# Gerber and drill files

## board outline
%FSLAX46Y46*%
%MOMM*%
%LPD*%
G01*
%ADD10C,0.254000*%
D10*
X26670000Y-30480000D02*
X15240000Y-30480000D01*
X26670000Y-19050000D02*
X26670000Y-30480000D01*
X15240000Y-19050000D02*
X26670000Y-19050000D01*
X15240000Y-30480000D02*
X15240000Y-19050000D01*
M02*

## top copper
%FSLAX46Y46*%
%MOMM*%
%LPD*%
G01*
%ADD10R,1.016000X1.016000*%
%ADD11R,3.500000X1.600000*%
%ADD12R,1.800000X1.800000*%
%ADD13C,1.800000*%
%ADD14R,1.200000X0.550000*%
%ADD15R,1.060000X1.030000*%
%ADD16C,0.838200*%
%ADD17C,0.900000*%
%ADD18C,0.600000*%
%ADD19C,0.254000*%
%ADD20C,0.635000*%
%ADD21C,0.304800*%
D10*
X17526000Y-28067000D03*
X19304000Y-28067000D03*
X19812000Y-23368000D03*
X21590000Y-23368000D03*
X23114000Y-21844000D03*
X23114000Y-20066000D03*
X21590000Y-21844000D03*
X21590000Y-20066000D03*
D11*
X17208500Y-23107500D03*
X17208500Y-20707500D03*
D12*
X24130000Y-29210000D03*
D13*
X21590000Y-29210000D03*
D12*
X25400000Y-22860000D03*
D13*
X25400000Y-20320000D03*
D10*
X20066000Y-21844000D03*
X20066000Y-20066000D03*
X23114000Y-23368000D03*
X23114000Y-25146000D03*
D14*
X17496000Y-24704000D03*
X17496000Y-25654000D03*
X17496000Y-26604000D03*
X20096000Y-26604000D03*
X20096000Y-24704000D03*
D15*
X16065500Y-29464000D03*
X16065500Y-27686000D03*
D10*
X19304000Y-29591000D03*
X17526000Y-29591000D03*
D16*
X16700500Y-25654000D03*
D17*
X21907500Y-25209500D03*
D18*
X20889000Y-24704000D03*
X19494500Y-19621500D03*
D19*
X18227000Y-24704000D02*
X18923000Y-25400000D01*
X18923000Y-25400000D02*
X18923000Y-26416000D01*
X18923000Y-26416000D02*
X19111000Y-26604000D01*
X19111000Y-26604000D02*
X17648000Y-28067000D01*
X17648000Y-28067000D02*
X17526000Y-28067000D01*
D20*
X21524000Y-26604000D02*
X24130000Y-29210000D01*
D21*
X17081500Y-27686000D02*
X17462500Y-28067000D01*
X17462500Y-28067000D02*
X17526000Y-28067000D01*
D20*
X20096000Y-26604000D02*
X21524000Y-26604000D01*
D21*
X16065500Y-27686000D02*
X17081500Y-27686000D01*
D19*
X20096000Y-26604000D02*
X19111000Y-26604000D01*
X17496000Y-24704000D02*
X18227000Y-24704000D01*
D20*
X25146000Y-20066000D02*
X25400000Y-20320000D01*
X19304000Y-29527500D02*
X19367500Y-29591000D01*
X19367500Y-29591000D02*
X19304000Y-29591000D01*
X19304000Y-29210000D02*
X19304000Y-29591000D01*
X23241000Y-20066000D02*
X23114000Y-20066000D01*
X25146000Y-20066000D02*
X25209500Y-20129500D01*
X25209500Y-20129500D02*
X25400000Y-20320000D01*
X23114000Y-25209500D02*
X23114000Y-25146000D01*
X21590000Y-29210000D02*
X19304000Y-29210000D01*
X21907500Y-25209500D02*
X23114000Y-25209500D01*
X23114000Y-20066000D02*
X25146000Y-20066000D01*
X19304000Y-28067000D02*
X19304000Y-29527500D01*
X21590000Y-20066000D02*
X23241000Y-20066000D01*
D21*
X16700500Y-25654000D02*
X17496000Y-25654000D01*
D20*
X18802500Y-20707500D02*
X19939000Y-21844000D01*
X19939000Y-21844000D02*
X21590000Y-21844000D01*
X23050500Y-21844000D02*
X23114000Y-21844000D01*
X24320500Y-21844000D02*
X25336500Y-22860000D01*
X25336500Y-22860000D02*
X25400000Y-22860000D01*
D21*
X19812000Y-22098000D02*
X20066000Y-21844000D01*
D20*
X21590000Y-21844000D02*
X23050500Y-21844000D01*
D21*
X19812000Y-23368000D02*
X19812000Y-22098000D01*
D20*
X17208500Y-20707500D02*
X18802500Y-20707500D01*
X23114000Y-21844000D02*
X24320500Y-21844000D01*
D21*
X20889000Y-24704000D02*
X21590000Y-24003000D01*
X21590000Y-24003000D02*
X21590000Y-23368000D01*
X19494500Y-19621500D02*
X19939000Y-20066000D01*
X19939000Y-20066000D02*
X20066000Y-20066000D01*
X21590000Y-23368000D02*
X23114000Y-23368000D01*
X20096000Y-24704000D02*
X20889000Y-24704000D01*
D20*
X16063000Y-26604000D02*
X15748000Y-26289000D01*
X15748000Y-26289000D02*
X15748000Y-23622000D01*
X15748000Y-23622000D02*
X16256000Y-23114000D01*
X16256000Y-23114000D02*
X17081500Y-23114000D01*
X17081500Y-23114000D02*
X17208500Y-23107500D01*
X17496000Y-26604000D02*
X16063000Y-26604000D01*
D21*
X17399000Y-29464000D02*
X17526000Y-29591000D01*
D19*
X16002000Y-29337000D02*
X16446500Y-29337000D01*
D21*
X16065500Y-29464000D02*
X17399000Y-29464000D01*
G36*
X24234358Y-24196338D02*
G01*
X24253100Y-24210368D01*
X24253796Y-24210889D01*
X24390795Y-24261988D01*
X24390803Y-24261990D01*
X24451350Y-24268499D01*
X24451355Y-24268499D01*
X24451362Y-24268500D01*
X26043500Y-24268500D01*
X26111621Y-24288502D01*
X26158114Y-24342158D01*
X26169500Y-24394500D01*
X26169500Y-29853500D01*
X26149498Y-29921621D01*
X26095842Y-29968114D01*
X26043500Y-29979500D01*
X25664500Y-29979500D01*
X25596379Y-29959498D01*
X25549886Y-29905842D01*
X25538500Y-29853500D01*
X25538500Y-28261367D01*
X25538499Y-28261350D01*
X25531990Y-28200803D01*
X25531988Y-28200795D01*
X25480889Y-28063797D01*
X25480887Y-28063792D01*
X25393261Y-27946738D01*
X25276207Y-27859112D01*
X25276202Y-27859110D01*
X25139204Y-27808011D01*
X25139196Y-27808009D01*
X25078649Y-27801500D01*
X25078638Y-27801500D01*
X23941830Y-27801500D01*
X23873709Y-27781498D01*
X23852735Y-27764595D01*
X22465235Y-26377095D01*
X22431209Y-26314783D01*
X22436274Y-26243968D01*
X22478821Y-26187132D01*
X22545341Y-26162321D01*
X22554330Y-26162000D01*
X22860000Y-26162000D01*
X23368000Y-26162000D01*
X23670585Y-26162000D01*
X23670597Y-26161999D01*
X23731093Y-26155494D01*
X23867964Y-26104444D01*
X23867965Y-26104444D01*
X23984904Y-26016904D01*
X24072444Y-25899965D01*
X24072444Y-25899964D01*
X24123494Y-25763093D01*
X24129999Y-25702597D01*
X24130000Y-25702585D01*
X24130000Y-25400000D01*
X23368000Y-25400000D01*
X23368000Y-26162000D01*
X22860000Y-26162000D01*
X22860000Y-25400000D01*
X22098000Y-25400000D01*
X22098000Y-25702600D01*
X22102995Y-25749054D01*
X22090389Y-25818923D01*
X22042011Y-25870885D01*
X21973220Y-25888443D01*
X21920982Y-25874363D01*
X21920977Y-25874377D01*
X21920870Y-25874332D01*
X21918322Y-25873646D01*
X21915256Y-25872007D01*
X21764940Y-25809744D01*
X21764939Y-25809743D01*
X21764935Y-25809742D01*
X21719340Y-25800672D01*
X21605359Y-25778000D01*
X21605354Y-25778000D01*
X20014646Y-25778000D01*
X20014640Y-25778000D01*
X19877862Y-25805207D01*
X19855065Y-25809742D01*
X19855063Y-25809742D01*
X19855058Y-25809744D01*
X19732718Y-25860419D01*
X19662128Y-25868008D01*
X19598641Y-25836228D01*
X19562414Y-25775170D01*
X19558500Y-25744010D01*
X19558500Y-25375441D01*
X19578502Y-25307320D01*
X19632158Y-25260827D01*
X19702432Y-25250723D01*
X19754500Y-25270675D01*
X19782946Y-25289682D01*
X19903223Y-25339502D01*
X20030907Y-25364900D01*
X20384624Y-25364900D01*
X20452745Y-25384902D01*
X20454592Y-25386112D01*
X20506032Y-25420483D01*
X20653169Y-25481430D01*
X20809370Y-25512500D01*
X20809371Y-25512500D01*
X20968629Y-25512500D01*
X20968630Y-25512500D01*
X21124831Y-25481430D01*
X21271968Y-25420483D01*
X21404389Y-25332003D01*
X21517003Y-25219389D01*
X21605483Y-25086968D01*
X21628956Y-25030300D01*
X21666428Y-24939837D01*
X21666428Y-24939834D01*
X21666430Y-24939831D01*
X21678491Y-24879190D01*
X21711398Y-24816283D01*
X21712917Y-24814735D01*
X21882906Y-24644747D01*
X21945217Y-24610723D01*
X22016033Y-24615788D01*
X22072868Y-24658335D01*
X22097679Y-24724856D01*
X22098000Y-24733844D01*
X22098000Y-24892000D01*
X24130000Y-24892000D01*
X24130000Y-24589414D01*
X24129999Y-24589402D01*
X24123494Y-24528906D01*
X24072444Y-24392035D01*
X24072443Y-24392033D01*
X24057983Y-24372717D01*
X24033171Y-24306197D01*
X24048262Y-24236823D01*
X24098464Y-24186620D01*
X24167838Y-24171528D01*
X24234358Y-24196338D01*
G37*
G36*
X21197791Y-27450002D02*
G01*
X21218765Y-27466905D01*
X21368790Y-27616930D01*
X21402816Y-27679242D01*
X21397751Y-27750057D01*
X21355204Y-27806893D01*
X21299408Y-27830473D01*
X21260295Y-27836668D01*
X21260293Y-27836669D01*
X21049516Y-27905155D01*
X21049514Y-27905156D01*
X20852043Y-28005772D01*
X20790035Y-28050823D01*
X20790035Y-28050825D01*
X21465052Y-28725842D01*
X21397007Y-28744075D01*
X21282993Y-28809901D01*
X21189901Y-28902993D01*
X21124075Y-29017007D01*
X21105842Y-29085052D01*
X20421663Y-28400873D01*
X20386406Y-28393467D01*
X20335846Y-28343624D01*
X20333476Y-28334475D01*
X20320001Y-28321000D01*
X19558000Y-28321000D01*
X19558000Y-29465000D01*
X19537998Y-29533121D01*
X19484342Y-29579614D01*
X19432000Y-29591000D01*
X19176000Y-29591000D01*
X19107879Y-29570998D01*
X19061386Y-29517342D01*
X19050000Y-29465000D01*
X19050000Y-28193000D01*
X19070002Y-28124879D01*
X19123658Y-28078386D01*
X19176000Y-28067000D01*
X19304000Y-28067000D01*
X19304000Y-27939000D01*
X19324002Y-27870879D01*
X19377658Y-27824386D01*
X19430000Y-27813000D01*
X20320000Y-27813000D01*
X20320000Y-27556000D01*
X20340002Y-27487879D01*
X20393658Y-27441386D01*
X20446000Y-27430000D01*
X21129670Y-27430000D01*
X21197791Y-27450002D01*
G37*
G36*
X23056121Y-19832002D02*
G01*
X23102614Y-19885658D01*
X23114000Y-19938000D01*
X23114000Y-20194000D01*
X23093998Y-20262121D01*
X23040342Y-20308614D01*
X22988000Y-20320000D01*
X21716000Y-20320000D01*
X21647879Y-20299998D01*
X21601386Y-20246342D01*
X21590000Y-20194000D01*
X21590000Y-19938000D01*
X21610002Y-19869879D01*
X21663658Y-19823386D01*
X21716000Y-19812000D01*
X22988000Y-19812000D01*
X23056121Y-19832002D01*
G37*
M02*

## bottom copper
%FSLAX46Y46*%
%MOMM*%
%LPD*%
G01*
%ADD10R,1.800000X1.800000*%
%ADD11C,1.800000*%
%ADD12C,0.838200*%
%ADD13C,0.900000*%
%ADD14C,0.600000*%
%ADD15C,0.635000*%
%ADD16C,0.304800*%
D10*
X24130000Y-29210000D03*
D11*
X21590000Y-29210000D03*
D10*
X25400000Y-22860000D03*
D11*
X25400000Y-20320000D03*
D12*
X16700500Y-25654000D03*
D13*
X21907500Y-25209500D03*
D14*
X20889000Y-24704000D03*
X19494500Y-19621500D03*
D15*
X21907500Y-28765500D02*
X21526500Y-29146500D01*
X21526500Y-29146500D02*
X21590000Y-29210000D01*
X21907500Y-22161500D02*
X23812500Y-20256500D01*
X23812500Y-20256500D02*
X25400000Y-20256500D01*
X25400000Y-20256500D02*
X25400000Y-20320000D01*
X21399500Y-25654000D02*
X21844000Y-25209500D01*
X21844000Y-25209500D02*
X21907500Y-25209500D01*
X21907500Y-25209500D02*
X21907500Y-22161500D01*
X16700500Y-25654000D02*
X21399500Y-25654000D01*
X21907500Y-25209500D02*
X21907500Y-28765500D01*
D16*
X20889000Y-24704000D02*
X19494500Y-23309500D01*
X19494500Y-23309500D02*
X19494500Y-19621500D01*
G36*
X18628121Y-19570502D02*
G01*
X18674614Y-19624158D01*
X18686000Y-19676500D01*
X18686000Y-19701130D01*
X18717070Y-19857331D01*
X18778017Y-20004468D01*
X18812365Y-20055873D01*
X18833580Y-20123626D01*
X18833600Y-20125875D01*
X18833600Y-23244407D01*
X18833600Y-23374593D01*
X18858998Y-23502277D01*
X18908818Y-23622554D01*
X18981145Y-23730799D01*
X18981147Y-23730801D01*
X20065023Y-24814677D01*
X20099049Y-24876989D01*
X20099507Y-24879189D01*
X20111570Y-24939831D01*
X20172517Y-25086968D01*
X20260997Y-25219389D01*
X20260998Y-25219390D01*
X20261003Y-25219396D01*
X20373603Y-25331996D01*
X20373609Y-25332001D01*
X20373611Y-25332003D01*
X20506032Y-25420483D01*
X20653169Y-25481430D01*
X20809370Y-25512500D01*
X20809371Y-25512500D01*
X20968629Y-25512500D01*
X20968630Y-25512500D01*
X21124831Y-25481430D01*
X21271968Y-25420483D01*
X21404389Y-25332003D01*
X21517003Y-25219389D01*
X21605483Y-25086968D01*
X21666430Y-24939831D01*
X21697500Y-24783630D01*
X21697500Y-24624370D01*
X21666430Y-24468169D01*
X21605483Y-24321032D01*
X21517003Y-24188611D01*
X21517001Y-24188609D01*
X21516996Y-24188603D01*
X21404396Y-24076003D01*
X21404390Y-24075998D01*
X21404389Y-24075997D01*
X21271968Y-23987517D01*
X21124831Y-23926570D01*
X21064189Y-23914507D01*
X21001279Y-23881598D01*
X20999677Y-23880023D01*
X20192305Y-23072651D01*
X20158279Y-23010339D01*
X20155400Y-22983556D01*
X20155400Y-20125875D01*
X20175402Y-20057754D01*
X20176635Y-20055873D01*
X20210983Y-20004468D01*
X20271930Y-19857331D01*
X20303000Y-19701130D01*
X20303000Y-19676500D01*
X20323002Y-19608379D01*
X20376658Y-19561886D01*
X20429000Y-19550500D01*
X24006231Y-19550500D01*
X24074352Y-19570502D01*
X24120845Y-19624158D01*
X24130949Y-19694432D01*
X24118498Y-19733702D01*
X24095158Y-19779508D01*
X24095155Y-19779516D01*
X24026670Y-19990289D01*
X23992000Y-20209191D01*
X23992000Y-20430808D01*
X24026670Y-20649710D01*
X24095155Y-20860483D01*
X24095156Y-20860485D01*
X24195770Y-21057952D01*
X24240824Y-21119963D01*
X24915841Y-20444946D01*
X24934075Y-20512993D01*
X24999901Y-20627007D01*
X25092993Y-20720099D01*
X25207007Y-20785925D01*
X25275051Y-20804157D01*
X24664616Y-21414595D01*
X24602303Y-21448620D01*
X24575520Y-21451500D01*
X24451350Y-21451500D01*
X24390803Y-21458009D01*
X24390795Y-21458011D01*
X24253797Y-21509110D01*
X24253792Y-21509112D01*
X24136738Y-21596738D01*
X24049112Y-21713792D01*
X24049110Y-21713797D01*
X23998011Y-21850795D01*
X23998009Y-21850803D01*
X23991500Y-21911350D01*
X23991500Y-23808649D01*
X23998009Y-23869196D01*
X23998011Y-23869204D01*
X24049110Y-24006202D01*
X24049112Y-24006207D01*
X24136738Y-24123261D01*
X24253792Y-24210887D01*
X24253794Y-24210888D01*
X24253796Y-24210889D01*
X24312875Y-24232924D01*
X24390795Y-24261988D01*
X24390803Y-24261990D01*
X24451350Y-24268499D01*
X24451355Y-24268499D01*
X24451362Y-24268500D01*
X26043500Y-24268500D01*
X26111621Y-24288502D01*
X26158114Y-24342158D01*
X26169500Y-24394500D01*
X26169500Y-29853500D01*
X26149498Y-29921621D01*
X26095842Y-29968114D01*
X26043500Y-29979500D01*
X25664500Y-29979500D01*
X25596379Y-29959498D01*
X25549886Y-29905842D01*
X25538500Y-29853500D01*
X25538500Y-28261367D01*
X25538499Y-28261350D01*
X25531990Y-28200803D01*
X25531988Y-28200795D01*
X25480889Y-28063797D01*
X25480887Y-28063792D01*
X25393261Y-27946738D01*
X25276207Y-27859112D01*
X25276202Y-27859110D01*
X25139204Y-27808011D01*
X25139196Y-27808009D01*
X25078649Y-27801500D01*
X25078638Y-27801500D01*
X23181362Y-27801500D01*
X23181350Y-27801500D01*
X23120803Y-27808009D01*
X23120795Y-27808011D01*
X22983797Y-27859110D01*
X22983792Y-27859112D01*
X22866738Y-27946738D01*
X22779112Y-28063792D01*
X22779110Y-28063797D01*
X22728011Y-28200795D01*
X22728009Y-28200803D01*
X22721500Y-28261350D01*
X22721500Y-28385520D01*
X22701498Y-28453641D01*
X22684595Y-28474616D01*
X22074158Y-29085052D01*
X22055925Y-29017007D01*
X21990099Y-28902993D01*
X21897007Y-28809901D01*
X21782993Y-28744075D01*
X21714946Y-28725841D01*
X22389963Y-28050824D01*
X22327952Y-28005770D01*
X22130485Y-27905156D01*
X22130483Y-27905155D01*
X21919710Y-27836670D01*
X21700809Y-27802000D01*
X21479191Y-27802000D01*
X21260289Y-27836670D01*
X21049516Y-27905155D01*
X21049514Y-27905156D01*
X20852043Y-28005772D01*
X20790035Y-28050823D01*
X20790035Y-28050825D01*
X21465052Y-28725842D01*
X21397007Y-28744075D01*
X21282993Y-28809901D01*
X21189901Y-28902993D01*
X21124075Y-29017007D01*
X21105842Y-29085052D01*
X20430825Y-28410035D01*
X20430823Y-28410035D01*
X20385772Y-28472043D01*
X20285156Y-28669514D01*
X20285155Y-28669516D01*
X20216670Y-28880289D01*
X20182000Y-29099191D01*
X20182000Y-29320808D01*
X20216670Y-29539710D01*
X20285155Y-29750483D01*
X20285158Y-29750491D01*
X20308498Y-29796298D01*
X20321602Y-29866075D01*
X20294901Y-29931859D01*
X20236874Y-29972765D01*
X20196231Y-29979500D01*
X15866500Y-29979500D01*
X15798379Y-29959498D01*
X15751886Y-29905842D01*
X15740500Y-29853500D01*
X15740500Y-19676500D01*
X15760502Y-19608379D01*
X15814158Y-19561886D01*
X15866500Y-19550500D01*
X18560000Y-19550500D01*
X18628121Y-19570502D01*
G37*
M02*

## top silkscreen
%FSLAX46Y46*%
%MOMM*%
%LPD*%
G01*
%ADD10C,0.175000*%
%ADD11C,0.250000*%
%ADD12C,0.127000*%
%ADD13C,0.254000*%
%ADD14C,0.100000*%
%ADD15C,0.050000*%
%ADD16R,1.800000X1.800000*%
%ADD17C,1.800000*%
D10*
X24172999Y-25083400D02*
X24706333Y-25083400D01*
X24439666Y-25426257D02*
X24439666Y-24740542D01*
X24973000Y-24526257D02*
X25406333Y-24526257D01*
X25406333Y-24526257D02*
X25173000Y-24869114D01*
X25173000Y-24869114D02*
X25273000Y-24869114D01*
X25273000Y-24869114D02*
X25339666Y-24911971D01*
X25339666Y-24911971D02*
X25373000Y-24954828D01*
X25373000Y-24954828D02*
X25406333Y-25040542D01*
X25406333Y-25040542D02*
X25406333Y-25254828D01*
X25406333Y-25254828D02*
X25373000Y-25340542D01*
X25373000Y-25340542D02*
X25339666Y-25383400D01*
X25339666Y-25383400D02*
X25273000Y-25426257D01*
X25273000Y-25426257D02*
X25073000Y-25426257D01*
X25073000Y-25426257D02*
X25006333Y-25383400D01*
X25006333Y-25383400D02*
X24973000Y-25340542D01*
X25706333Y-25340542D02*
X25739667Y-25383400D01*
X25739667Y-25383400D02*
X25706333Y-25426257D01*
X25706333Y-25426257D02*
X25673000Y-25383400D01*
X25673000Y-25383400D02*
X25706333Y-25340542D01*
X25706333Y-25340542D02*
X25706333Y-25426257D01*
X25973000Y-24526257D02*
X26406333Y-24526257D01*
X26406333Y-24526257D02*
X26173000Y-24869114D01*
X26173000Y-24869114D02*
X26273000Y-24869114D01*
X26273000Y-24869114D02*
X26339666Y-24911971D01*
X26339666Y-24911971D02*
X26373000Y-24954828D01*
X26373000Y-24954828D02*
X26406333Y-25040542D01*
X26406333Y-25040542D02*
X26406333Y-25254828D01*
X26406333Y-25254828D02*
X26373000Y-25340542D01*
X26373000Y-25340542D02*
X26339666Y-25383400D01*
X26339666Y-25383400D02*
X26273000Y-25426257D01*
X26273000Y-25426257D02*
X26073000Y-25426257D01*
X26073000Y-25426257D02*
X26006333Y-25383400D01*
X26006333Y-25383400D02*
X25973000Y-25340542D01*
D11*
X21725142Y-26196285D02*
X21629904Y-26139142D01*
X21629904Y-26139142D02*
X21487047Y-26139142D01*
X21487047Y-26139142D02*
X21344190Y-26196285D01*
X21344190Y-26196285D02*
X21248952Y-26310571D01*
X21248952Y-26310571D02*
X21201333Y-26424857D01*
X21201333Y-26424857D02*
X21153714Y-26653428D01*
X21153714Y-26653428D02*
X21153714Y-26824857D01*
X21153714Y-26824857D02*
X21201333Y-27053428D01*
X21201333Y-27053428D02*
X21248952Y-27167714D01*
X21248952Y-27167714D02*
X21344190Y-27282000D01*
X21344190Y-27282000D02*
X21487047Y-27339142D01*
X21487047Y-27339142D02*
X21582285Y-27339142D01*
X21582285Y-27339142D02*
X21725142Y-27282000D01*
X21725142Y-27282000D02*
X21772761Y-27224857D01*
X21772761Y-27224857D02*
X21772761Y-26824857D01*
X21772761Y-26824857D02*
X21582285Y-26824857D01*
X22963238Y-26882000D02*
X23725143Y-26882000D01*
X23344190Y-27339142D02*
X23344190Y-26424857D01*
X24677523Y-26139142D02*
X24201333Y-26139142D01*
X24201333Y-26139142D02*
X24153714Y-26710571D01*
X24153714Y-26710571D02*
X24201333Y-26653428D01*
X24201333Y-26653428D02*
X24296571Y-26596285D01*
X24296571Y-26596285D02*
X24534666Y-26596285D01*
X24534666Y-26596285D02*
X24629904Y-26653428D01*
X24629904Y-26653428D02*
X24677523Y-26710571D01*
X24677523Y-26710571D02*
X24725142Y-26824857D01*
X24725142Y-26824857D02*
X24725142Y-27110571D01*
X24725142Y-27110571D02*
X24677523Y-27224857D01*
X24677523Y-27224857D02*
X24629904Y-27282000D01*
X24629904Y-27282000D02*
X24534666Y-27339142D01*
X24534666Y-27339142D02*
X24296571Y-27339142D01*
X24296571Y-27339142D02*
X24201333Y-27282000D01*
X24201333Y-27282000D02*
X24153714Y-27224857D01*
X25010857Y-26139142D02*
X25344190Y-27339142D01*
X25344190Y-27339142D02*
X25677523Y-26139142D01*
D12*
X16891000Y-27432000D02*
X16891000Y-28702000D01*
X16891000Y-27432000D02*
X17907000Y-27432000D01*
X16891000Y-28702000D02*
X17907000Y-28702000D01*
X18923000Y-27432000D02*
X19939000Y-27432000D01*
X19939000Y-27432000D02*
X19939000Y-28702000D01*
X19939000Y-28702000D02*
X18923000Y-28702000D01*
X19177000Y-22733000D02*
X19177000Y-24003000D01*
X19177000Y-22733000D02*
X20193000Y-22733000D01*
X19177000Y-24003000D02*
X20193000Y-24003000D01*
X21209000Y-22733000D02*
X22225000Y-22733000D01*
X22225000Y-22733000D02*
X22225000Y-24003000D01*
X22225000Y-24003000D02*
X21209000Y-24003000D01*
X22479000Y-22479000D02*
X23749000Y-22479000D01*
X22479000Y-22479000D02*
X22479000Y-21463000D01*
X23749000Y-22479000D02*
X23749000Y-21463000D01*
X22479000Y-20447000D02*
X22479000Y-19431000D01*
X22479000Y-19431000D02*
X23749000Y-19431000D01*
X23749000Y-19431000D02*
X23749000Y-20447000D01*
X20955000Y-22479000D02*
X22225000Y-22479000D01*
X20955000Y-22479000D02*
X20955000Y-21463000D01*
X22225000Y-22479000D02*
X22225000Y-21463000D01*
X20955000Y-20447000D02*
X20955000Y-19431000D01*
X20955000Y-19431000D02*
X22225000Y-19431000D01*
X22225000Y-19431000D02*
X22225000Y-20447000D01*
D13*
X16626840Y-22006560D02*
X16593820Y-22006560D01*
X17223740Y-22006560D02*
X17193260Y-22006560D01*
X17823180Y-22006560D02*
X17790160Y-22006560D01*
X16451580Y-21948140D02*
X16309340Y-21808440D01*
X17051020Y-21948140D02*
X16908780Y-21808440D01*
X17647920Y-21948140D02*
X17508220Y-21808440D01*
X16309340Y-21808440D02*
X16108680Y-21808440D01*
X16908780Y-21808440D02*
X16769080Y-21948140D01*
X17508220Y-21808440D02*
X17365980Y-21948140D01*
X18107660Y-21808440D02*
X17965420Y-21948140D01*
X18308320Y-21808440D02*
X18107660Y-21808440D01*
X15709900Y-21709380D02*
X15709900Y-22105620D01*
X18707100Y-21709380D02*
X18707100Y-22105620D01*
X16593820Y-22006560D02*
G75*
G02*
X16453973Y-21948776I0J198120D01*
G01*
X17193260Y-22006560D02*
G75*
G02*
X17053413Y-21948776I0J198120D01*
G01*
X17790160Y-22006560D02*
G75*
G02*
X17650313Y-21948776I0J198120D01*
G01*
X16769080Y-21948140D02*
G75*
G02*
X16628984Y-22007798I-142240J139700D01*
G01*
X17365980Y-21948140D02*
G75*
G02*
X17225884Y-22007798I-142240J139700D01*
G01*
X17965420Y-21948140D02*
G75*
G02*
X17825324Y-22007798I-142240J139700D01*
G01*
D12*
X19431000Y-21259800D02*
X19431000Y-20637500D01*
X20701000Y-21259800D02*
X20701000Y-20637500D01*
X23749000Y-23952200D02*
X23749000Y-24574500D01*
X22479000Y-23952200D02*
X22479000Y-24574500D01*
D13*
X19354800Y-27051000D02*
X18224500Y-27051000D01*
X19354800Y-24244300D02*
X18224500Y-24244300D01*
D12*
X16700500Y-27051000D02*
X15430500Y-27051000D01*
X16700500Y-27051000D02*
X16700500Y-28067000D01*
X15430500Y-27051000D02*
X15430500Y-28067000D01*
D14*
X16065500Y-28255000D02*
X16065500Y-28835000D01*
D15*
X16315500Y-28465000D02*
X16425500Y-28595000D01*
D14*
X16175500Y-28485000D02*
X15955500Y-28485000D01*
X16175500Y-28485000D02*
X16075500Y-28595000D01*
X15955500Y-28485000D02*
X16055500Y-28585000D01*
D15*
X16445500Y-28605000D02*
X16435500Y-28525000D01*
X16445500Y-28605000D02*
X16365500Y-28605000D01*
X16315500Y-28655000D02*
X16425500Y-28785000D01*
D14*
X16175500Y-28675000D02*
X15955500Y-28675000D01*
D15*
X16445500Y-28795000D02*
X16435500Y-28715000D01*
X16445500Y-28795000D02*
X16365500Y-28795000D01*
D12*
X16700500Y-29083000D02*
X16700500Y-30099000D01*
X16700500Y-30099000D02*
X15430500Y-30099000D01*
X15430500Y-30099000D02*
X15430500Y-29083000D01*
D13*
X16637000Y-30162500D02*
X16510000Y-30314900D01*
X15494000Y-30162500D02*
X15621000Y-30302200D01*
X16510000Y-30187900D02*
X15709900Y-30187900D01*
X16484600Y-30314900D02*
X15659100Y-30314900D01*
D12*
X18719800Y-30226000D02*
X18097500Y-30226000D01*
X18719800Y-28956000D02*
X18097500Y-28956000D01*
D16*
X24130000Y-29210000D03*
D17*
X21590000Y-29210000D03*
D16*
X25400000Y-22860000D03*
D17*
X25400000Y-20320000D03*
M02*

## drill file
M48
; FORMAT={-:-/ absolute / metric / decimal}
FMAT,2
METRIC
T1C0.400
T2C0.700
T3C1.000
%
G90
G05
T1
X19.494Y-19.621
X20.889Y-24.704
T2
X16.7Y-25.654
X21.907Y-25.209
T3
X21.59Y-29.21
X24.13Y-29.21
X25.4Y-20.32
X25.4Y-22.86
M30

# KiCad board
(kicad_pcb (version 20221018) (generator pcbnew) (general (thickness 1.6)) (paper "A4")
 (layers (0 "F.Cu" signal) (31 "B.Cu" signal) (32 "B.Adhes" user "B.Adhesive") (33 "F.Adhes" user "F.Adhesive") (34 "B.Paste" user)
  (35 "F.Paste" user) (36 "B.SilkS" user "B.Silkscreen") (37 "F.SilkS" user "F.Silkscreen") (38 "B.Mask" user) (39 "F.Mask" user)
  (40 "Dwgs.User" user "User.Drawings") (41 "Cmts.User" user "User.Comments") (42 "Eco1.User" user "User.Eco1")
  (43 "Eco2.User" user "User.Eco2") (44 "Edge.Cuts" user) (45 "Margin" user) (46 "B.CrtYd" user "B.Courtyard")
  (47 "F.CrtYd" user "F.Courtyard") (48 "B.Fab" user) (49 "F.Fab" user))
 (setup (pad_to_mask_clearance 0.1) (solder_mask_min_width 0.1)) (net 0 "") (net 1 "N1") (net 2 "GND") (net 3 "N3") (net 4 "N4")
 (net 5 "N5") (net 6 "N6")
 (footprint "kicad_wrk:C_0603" (layer "F.Cu") (at 18.415 28.067)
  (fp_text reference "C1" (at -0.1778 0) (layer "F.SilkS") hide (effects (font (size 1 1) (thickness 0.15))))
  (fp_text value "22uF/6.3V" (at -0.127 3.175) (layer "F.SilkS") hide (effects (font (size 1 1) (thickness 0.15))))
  (fp_line (start -1.524 -0.635) (end -1.524 0.635) (stroke (width 0.127) (type solid)) (layer "F.SilkS"))
  (fp_line (start -1.524 -0.635) (end -0.508 -0.635) (stroke (width 0.127) (type solid)) (layer "F.SilkS"))
  (fp_line (start -1.524 0.635) (end -0.508 0.635) (stroke (width 0.127) (type solid)) (layer "F.SilkS"))
  (fp_line (start 0.508 -0.635) (end 1.524 -0.635) (stroke (width 0.127) (type solid)) (layer "F.SilkS"))
  (fp_line (start 1.524 -0.635) (end 1.524 0.635) (stroke (width 0.127) (type solid)) (layer "F.SilkS"))
  (fp_line (start 1.524 0.635) (end 0.508 0.635) (stroke (width 0.127) (type solid)) (layer "F.SilkS"))
  (pad "1" smd rect (at -0.889 0) (size 1.016 1.016) (layers "F.Cu" "F.Paste" "F.Mask") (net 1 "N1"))
  (pad "2" smd rect (at 0.889 0) (size 1.016 1.016) (layers "F.Cu" "F.Paste" "F.Mask") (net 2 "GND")))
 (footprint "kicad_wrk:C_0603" (layer "F.Cu") (at 20.701 23.368)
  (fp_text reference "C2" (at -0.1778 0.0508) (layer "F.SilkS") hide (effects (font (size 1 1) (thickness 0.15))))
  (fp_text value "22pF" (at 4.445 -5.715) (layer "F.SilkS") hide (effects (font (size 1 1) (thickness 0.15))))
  (fp_line (start -1.524 -0.635) (end -1.524 0.635) (stroke (width 0.127) (type solid)) (layer "F.SilkS"))
  (fp_line (start -1.524 -0.635) (end -0.508 -0.635) (stroke (width 0.127) (type solid)) (layer "F.SilkS"))
  (fp_line (start -1.524 0.635) (end -0.508 0.635) (stroke (width 0.127) (type solid)) (layer "F.SilkS"))
  (fp_line (start 0.508 -0.635) (end 1.524 -0.635) (stroke (width 0.127) (type solid)) (layer "F.SilkS"))
  (fp_line (start 1.524 -0.635) (end 1.524 0.635) (stroke (width 0.127) (type solid)) (layer "F.SilkS"))
  (fp_line (start 1.524 0.635) (end 0.508 0.635) (stroke (width 0.127) (type solid)) (layer "F.SilkS"))
  (pad "1" smd rect (at -0.889 0) (size 1.016 1.016) (layers "F.Cu" "F.Paste" "F.Mask") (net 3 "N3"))
  (pad "2" smd rect (at 0.889 0) (size 1.016 1.016) (layers "F.Cu" "F.Paste" "F.Mask") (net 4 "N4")))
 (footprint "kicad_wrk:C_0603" (layer "F.Cu") (at 23.114 20.955 90)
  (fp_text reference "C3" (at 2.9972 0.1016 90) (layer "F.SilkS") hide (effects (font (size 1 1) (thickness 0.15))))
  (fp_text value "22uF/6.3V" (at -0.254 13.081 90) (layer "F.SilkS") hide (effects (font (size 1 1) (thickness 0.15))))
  (fp_line (start -1.524 -0.635) (end -1.524 0.635) (stroke (width 0.127) (type solid)) (layer "F.SilkS"))
  (fp_line (start -1.524 -0.635) (end -0.508 -0.635) (stroke (width 0.127) (type solid)) (layer "F.SilkS"))
  (fp_line (start -1.524 0.635) (end -0.508 0.635) (stroke (width 0.127) (type solid)) (layer "F.SilkS"))
  (fp_line (start 0.508 -0.635) (end 1.524 -0.635) (stroke (width 0.127) (type solid)) (layer "F.SilkS"))
  (fp_line (start 1.524 -0.635) (end 1.524 0.635) (stroke (width 0.127) (type solid)) (layer "F.SilkS"))
  (fp_line (start 1.524 0.635) (end 0.508 0.635) (stroke (width 0.127) (type solid)) (layer "F.SilkS"))
  (pad "1" smd rect (at -0.889 0 90) (size 1.016 1.016) (layers "F.Cu" "F.Paste" "F.Mask") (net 3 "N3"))
  (pad "2" smd rect (at 0.889 0 90) (size 1.016 1.016) (layers "F.Cu" "F.Paste" "F.Mask") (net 2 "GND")))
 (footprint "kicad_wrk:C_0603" (layer "F.Cu") (at 21.59 20.955 90)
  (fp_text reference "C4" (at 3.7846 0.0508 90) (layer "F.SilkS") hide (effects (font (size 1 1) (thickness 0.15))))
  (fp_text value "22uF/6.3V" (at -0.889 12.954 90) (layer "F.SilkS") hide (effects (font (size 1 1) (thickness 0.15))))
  (fp_line (start -1.524 -0.635) (end -1.524 0.635) (stroke (width 0.127) (type solid)) (layer "F.SilkS"))
  (fp_line (start -1.524 -0.635) (end -0.508 -0.635) (stroke (width 0.127) (type solid)) (layer "F.SilkS"))
  (fp_line (start -1.524 0.635) (end -0.508 0.635) (stroke (width 0.127) (type solid)) (layer "F.SilkS"))
  (fp_line (start 0.508 -0.635) (end 1.524 -0.635) (stroke (width 0.127) (type solid)) (layer "F.SilkS"))
  (fp_line (start 1.524 -0.635) (end 1.524 0.635) (stroke (width 0.127) (type solid)) (layer "F.SilkS"))
  (fp_line (start 1.524 0.635) (end 0.508 0.635) (stroke (width 0.127) (type solid)) (layer "F.SilkS"))
  (pad "1" smd rect (at -0.889 0 90) (size 1.016 1.016) (layers "F.Cu" "F.Paste" "F.Mask") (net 3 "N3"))
  (pad "2" smd rect (at 0.889 0 90) (size 1.016 1.016) (layers "F.Cu" "F.Paste" "F.Mask") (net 2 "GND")))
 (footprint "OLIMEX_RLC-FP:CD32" (layer "F.Cu") (at 17.2085 21.9075 90)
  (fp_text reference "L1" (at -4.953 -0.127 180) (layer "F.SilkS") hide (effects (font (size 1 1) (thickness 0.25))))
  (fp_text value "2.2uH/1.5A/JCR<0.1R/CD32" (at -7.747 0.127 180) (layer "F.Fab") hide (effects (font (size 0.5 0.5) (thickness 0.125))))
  (fp_line (start -0.09906 -0.58166) (end -0.09906 -0.61468) (stroke (width 0.254) (type solid)) (layer "F.SilkS"))
  (fp_line (start -0.09906 0.01524) (end -0.09906 -0.01524) (stroke (width 0.254) (type solid)) (layer "F.SilkS"))
  (fp_line (start -0.09906 0.61468) (end -0.09906 0.58166) (stroke (width 0.254) (type solid)) (layer "F.SilkS"))
  (fp_line (start -0.04064 -0.75692) (end 0.09906 -0.89916) (stroke (width 0.254) (type solid)) (layer "F.SilkS"))
  (fp_line (start -0.04064 -0.15748) (end 0.09906 -0.29972) (stroke (width 0.254) (type solid)) (layer "F.SilkS"))
  (fp_line (start -0.04064 0.43942) (end 0.09906 0.29972) (stroke (width 0.254) (type solid)) (layer "F.SilkS"))
  (fp_line (start 0.09906 -0.89916) (end 0.09906 -1.09982) (stroke (width 0.254) (type solid)) (layer "F.SilkS"))
  (fp_line (start 0.09906 -0.29972) (end -0.04064 -0.43942) (stroke (width 0.254) (type solid)) (layer "F.SilkS"))
  (fp_line (start 0.09906 0.29972) (end -0.04064 0.15748) (stroke (width 0.254) (type solid)) (layer "F.SilkS"))
  (fp_line (start 0.09906 0.89916) (end -0.04064 0.75692) (stroke (width 0.254) (type solid)) (layer "F.SilkS"))
  (fp_line (start 0.09906 1.09982) (end 0.09906 0.89916) (stroke (width 0.254) (type solid)) (layer "F.SilkS"))
  (fp_line (start 0.19812 -1.4986) (end -0.19812 -1.4986) (stroke (width 0.254) (type solid)) (layer "F.SilkS"))
  (fp_line (start 0.19812 1.4986) (end -0.19812 1.4986) (stroke (width 0.254) (type solid)) (layer "F.SilkS"))
  (fp_arc (start -0.09906 -0.61468) (mid -0.084045 -0.690337) (end -0.041276 -0.754527) (stroke (width 0.254) (type solid))
   (layer "F.SilkS"))
  (fp_arc (start -0.09906 -0.01524) (mid -0.084045 -0.090897) (end -0.041276 -0.155087) (stroke (width 0.254) (type solid))
   (layer "F.SilkS"))
  (fp_arc (start -0.09906 0.58166) (mid -0.084045 0.506003) (end -0.041276 0.441813) (stroke (width 0.254) (type solid)) (layer "F.SilkS"))
  (fp_arc (start -0.04064 -0.43942) (mid -0.084371 -0.503548) (end -0.100298 -0.579516) (stroke (width 0.254) (type solid))
   (layer "F.SilkS"))
  (fp_arc (start -0.04064 0.15748) (mid -0.084371 0.093352) (end -0.100298 0.017384) (stroke (width 0.254) (type solid)) (layer "F.SilkS"))
  (fp_arc (start -0.04064 0.75692) (mid -0.084371 0.692792) (end -0.100298 0.616824) (stroke (width 0.254) (type solid)) (layer "F.SilkS"))
  (pad "1" smd rect (at -1.2 0 180) (size 3.5 1.6) (layers "F.Cu" "F.Paste" "F.Mask") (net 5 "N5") (solder_mask_margin 0.0508)
   (solder_paste_margin -0.0508) (clearance 0.0508))
  (pad "2" smd rect (at 1.2 0 180) (size 3.5 1.6) (layers "F.Cu" "F.Paste" "F.Mask") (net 3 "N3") (solder_mask_margin 0.0508)
   (solder_paste_margin -0.0508) (clearance 0.0508)))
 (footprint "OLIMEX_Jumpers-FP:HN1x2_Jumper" (layer "F.Cu") (at 22.86 29.21 180)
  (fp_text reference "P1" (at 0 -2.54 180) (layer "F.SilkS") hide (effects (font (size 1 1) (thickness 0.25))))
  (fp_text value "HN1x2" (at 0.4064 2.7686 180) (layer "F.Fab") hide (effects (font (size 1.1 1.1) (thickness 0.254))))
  (pad "1" thru_hole rect (at -1.27 0 270) (size 1.8 1.8) (drill 1) (layers "*.Cu" "*.Mask" "F.SilkS") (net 1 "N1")
   (solder_mask_margin 0.0508) (solder_paste_margin -0.0508))
  (pad "2" thru_hole circle (at 1.27 0 270) (size 1.8 1.8) (drill 1) (layers "*.Cu" "*.Mask" "F.SilkS") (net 2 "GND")
   (solder_mask_margin 0.0508) (solder_paste_margin -0.0508)))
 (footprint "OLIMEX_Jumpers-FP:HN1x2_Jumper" (layer "F.Cu") (at 25.4 21.59 90)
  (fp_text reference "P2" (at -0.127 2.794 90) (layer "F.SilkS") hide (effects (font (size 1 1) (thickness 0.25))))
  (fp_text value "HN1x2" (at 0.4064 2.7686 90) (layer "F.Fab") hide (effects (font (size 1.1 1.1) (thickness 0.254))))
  (pad "1" thru_hole rect (at -1.27 0 180) (size 1.8 1.8) (drill 1) (layers "*.Cu" "*.Mask" "F.SilkS") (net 3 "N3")
   (solder_mask_margin 0.0508) (solder_paste_margin -0.0508))
  (pad "2" thru_hole circle (at 1.27 0 180) (size 1.8 1.8) (drill 1) (layers "*.Cu" "*.Mask" "F.SilkS") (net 2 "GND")
   (solder_mask_margin 0.0508) (solder_paste_margin -0.0508)))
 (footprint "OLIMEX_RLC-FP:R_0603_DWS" (layer "F.Cu") (at 20.066 20.955 90)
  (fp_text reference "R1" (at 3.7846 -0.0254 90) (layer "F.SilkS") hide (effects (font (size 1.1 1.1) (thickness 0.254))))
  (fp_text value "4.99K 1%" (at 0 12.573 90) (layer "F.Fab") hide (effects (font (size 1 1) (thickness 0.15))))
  (fp_line (start -0.3048 -0.635) (end 0.3175 -0.635) (stroke (width 0.127) (type solid)) (layer "F.SilkS"))
  (fp_line (start -0.3048 0.635) (end 0.3175 0.635) (stroke (width 0.127) (type solid)) (layer "F.SilkS"))
  (pad "1" smd rect (at -0.889 0 90) (size 1.016 1.016) (layers "F.Cu" "F.Paste" "F.Mask") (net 3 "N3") (solder_mask_margin 0.0508)
   (solder_paste_margin -0.0508) (clearance 0.0508))
  (pad "2" smd rect (at 0.889 0 90) (size 1.016 1.016) (layers "F.Cu" "F.Paste" "F.Mask") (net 4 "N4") (solder_mask_margin 0.0508)
   (solder_paste_margin -0.0508) (clearance 0.0508)))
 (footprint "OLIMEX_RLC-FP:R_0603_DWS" (layer "F.Cu") (at 23.114 24.257 -90)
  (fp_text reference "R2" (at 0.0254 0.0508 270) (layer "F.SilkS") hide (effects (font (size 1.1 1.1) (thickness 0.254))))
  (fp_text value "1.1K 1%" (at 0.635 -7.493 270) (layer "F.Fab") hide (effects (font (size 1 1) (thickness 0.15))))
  (fp_line (start -0.3048 -0.635) (end 0.3175 -0.635) (stroke (width 0.127) (type solid)) (layer "F.SilkS"))
  (fp_line (start -0.3048 0.635) (end 0.3175 0.635) (stroke (width 0.127) (type solid)) (layer "F.SilkS"))
  (pad "1" smd rect (at -0.889 0 270) (size 1.016 1.016) (layers "F.Cu" "F.Paste" "F.Mask") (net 4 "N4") (solder_mask_margin 0.0508)
   (solder_paste_margin -0.0508) (clearance 0.0508))
  (pad "2" smd rect (at 0.889 0 270) (size 1.016 1.016) (layers "F.Cu" "F.Paste" "F.Mask") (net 2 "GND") (solder_mask_margin 0.0508)
   (solder_paste_margin -0.0508) (clearance 0.0508)))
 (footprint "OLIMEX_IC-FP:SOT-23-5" (layer "F.Cu") (at 18.796 25.654 180)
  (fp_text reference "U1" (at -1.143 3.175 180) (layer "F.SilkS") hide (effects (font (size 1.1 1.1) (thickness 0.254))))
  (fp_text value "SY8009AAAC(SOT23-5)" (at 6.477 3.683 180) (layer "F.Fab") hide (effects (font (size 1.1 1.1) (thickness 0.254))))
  (fp_line (start -0.5588 -1.397) (end 0.5715 -1.397) (stroke (width 0.254) (type solid)) (layer "F.SilkS"))
  (fp_line (start -0.5588 1.4097) (end 0.5715 1.4097) (stroke (width 0.254) (type solid)) (layer "F.SilkS"))
  (pad "1" smd rect (at 1.3 0.95 180) (size 1.2 0.55) (layers "F.Cu" "F.Paste" "F.Mask") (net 1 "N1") (solder_mask_margin 0.0508)
   (solder_paste_margin -0.0508) (clearance 0.0508))
  (pad "2" smd rect (at 1.3 0 180) (size 1.2 0.55) (layers "F.Cu" "F.Paste" "F.Mask") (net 2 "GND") (solder_mask_margin 0.0508)
   (solder_paste_margin -0.0508) (clearance 0.0508))
  (pad "3" smd rect (at 1.3 -0.95 180) (size 1.2 0.55) (layers "F.Cu" "F.Paste" "F.Mask") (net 5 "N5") (solder_mask_margin 0.0508)
   (solder_paste_margin -0.0508) (clearance 0.0508))
  (pad "4" smd rect (at -1.3 -0.95 180) (size 1.2 0.55) (layers "F.Cu" "F.Paste" "F.Mask") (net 1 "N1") (solder_mask_margin 0.0508)
   (solder_paste_margin -0.0508) (clearance 0.0508))
  (pad "5" smd rect (at -1.3 0.95 180) (size 1.2 0.55) (layers "F.Cu" "F.Paste" "F.Mask") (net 4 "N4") (solder_mask_margin 0.0508)
   (solder_paste_margin -0.0508) (clearance 0.0508)))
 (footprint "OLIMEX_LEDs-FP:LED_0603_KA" (layer "F.Cu") (at 16.0655 28.575 -90)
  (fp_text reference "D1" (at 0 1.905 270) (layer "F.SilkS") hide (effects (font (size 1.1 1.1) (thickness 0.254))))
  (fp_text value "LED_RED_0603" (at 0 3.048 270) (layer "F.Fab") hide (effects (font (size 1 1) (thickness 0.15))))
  (fp_line (start -1.524 -0.635) (end -1.524 0.635) (stroke (width 0.127) (type solid)) (layer "F.SilkS"))
  (fp_line (start -1.524 -0.635) (end -0.508 -0.635) (stroke (width 0.127) (type solid)) (layer "F.SilkS"))
  (fp_line (start -1.524 0.635) (end -0.508 0.635) (stroke (width 0.127) (type solid)) (layer "F.SilkS"))
  (fp_line (start -0.32 0) (end 0.26 0) (stroke (width 0.1) (type solid)) (layer "F.SilkS"))
  (fp_line (start -0.11 -0.25) (end 0.02 -0.36) (stroke (width 0.05) (type solid)) (layer "F.SilkS"))
  (fp_line (start -0.09 -0.11) (end -0.09 0.11) (stroke (width 0.1) (type solid)) (layer "F.SilkS"))
  (fp_line (start -0.09 -0.11) (end 0.02 -0.01) (stroke (width 0.1) (type solid)) (layer "F.SilkS"))
  (fp_line (start -0.09 0.11) (end 0.01 0.01) (stroke (width 0.1) (type solid)) (layer "F.SilkS"))
  (fp_line (start 0.03 -0.38) (end -0.05 -0.37) (stroke (width 0.05) (type solid)) (layer "F.SilkS"))
  (fp_line (start 0.03 -0.38) (end 0.03 -0.3) (stroke (width 0.05) (type solid)) (layer "F.SilkS"))
  (fp_line (start 0.08 -0.25) (end 0.21 -0.36) (stroke (width 0.05) (type solid)) (layer "F.SilkS"))
  (fp_line (start 0.1 -0.11) (end 0.1 0.11) (stroke (width 0.1) (type solid)) (layer "F.SilkS"))
  (fp_line (start 0.22 -0.38) (end 0.14 -0.37) (stroke (width 0.05) (type solid)) (layer "F.SilkS"))
  (fp_line (start 0.22 -0.38) (end 0.22 -0.3) (stroke (width 0.05) (type solid)) (layer "F.SilkS"))
  (fp_line (start 0.508 -0.635) (end 1.524 -0.635) (stroke (width 0.127) (type solid)) (layer "F.SilkS"))
  (fp_line (start 1.524 -0.635) (end 1.524 0.635) (stroke (width 0.127) (type solid)) (layer "F.SilkS"))
  (fp_line (start 1.524 0.635) (end 0.508 0.635) (stroke (width 0.127) (type solid)) (layer "F.SilkS"))
  (fp_line (start 1.5875 -0.5715) (end 1.7399 -0.4445) (stroke (width 0.254) (type solid)) (layer "F.SilkS"))
  (fp_line (start 1.5875 0.5715) (end 1.7272 0.4445) (stroke (width 0.254) (type solid)) (layer "F.SilkS"))
  (fp_line (start 1.6129 -0.4445) (end 1.6129 0.3556) (stroke (width 0.254) (type solid)) (layer "F.SilkS"))
  (fp_line (start 1.7399 -0.4191) (end 1.7399 0.4064) (stroke (width 0.254) (type solid)) (layer "F.SilkS"))
  (pad "1" smd rect (at 0.889 0 270) (size 1.03 1.06) (layers "F.Cu" "F.Paste" "F.Mask") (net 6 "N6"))
  (pad "2" smd rect (at -0.889 0 270) (size 1.03 1.06) (layers "F.Cu" "F.Paste" "F.Mask") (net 1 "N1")))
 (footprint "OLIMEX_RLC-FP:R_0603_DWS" (layer "F.Cu") (at 18.415 29.591 180)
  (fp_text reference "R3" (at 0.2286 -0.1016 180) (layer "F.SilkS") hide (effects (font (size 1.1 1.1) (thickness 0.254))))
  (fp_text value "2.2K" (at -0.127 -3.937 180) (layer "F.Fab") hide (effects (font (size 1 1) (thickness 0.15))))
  (fp_line (start -0.3048 -0.635) (end 0.3175 -0.635) (stroke (width 0.127) (type solid)) (layer "F.SilkS"))
  (fp_line (start -0.3048 0.635) (end 0.3175 0.635) (stroke (width 0.127) (type solid)) (layer "F.SilkS"))
  (pad "1" smd rect (at -0.889 0 180) (size 1.016 1.016) (layers "F.Cu" "F.Paste" "F.Mask") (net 2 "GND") (solder_mask_margin 0.0508)
   (solder_paste_margin -0.0508) (clearance 0.0508))
  (pad "2" smd rect (at 0.889 0 180) (size 1.016 1.016) (layers "F.Cu" "F.Paste" "F.Mask") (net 6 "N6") (solder_mask_margin 0.0508)
   (solder_paste_margin -0.0508) (clearance 0.0508)))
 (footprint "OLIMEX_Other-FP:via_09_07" (layer "F.Cu") (at 16.7005 25.654)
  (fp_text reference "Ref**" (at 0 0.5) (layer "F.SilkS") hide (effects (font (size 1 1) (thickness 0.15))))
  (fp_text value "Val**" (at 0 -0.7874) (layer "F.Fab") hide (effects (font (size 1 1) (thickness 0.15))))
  (pad "0" thru_hole circle (at 0 0) (size 0.8382 0.8382) (drill 0.7) (layers "*.Cu") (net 2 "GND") (zone_connect 2)))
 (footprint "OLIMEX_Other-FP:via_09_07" (layer "F.Cu") (at 21.9075 25.273)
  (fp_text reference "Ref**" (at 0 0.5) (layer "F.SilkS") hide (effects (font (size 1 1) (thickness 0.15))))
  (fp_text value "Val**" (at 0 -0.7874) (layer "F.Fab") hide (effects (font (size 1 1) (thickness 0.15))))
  (pad "0" thru_hole circle (at 0 -0.0635) (size 0.9 0.9) (drill 0.7) (layers "*.Cu") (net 2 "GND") (zone_connect 2)))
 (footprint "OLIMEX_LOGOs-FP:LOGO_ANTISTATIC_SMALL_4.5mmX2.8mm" (layer "B.Cu") (at 18.4785 28.194 180)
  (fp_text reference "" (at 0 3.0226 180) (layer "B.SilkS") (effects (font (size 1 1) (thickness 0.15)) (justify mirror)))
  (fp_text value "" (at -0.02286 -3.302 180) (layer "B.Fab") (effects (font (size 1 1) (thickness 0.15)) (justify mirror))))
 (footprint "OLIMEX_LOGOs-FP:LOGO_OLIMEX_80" (layer "B.Cu") (at 19.939 24.3205 180)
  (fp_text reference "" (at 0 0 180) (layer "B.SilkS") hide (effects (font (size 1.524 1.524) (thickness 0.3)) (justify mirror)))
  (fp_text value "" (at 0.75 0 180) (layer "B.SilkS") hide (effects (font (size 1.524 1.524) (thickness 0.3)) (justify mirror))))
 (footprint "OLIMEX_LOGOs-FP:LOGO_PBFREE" (layer "B.Cu") (at 18.669 21.3995 180)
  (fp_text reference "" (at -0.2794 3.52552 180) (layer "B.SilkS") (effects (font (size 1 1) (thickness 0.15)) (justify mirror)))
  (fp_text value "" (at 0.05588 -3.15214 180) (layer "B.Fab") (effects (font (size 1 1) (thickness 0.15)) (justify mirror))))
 (gr_line (start 26.67 30.48) (end 15.24 30.48) (stroke (width 0.254) (type solid)) (layer "Edge.Cuts"))
 (gr_line (start 26.67 19.05) (end 26.67 30.48) (stroke (width 0.254) (type solid)) (layer "Edge.Cuts"))
 (gr_line (start 15.24 19.05) (end 26.67 19.05) (stroke (width 0.254) (type solid)) (layer "Edge.Cuts"))
 (gr_line (start 15.24 30.48) (end 15.24 19.05) (stroke (width 0.254) (type solid)) (layer "Edge.Cuts"))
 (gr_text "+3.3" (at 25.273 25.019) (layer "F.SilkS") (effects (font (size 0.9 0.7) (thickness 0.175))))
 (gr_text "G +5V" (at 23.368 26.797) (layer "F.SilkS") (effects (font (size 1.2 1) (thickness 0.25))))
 (segment (start 18.227 24.704) (end 18.923 25.4) (width 0.254) (layer "F.Cu") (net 1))
 (segment (start 18.923 25.4) (end 18.923 26.416) (width 0.254) (layer "F.Cu") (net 1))
 (segment (start 18.923 26.416) (end 19.111 26.604) (width 0.254) (layer "F.Cu") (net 1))
 (segment (start 19.111 26.604) (end 17.648 28.067) (width 0.254) (layer "F.Cu") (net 1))
 (segment (start 17.648 28.067) (end 17.526 28.067) (width 0.254) (layer "F.Cu") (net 1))
 (segment (start 21.524 26.604) (end 24.13 29.21) (width 0.635) (layer "F.Cu") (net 1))
 (segment (start 17.0815 27.686) (end 17.4625 28.067) (width 0.3048) (layer "F.Cu") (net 1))
 (segment (start 17.4625 28.067) (end 17.526 28.067) (width 0.3048) (layer "F.Cu") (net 1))
 (segment (start 20.096 26.604) (end 21.524 26.604) (width 0.635) (layer "F.Cu") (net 1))
 (segment (start 16.0655 27.686) (end 17.0815 27.686) (width 0.3048) (layer "F.Cu") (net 1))
 (segment (start 20.096 26.604) (end 19.111 26.604) (width 0.254) (layer "F.Cu") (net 1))
 (segment (start 17.496 24.704) (end 18.227 24.704) (width 0.254) (layer "F.Cu") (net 1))
 (segment (start 25.146 20.066) (end 25.4 20.32) (width 0.635) (layer "F.Cu") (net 2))
 (segment (start 19.304 29.5275) (end 19.3675 29.591) (width 0.635) (layer "F.Cu") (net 2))
 (segment (start 19.3675 29.591) (end 19.304 29.591) (width 0.635) (layer "F.Cu") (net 2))
 (segment (start 19.304 29.21) (end 19.304 29.591) (width 0.635) (layer "F.Cu") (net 2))
 (segment (start 23.241 20.066) (end 23.114 20.066) (width 0.635) (layer "F.Cu") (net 2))
 (segment (start 25.146 20.066) (end 25.2095 20.1295) (width 0.635) (layer "F.Cu") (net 2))
 (segment (start 25.2095 20.1295) (end 25.4 20.32) (width 0.635) (layer "F.Cu") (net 2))
 (segment (start 23.114 25.2095) (end 23.114 25.146) (width 0.635) (layer "F.Cu") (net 2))
 (segment (start 21.59 29.21) (end 19.304 29.21) (width 0.635) (layer "F.Cu") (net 2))
 (segment (start 21.9075 25.2095) (end 23.114 25.2095) (width 0.635) (layer "F.Cu") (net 2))
 (segment (start 23.114 20.066) (end 25.146 20.066) (width 0.635) (layer "F.Cu") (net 2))
 (segment (start 19.304 28.067) (end 19.304 29.5275) (width 0.635) (layer "F.Cu") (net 2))
 (segment (start 21.59 20.066) (end 23.241 20.066) (width 0.635) (layer "F.Cu") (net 2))
 (segment (start 16.7005 25.654) (end 17.496 25.654) (width 0.3048) (layer "F.Cu") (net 2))
 (segment (start 21.9075 28.7655) (end 21.5265 29.1465) (width 0.635) (layer "B.Cu") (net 2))
 (segment (start 21.5265 29.1465) (end 21.59 29.21) (width 0.635) (layer "B.Cu") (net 2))
 (segment (start 21.9075 22.1615) (end 23.8125 20.2565) (width 0.635) (layer "B.Cu") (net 2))
 (segment (start 23.8125 20.2565) (end 25.4 20.2565) (width 0.635) (layer "B.Cu") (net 2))
 (segment (start 25.4 20.2565) (end 25.4 20.32) (width 0.635) (layer "B.Cu") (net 2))
 (segment (start 21.3995 25.654) (end 21.844 25.2095) (width 0.635) (layer "B.Cu") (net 2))
 (segment (start 21.844 25.2095) (end 21.9075 25.2095) (width 0.635) (layer "B.Cu") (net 2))
 (segment (start 21.9075 25.2095) (end 21.9075 22.1615) (width 0.635) (layer "B.Cu") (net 2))
 (segment (start 16.7005 25.654) (end 21.3995 25.654) (width 0.635) (layer "B.Cu") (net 2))
 (segment (start 21.9075 25.2095) (end 21.9075 28.7655) (width 0.635) (layer "B.Cu") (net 2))
 (segment (start 18.8025 20.7075) (end 19.939 21.844) (width 0.635) (layer "F.Cu") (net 3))
 (segment (start 19.939 21.844) (end 21.59 21.844) (width 0.635) (layer "F.Cu") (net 3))
 (segment (start 23.0505 21.844) (end 23.114 21.844) (width 0.635) (layer "F.Cu") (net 3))
 (segment (start 24.3205 21.844) (end 25.3365 22.86) (width 0.635) (layer "F.Cu") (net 3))
 (segment (start 25.3365 22.86) (end 25.4 22.86) (width 0.635) (layer "F.Cu") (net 3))
 (segment (start 19.812 22.098) (end 20.066 21.844) (width 0.3048) (layer "F.Cu") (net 3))
 (segment (start 21.59 21.844) (end 23.0505 21.844) (width 0.635) (layer "F.Cu") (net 3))
 (segment (start 19.812 23.368) (end 19.812 22.098) (width 0.3048) (layer "F.Cu") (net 3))
 (segment (start 17.2085 20.7075) (end 18.8025 20.7075) (width 0.635) (layer "F.Cu") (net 3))
 (segment (start 23.114 21.844) (end 24.3205 21.844) (width 0.635) (layer "F.Cu") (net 3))
 (segment (start 20.889 24.704) (end 21.59 24.003) (width 0.3048) (layer "F.Cu") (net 4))
 (segment (start 21.59 24.003) (end 21.59 23.368) (width 0.3048) (layer "F.Cu") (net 4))
 (segment (start 19.4945 19.6215) (end 19.939 20.066) (width 0.3048) (layer "F.Cu") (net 4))
 (segment (start 19.939 20.066) (end 20.066 20.066) (width 0.3048) (layer "F.Cu") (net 4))
 (segment (start 21.59 23.368) (end 23.114 23.368) (width 0.3048) (layer "F.Cu") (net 4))
 (segment (start 20.096 24.704) (end 20.889 24.704) (width 0.3048) (layer "F.Cu") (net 4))
 (via (at 20.889 24.704) (size 0.6) (drill 0.4) (layers "F.Cu" "B.Cu") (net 4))
 (via (at 19.4945 19.6215) (size 0.6) (drill 0.4) (layers "F.Cu" "B.Cu") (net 4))
 (segment (start 20.889 24.704) (end 19.4945 23.3095) (width 0.3048) (layer "B.Cu") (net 4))
 (segment (start 19.4945 23.3095) (end 19.4945 19.6215) (width 0.3048) (layer "B.Cu") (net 4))
 (segment (start 16.063 26.604) (end 15.748 26.289) (width 0.635) (layer "F.Cu") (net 5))
 (segment (start 15.748 26.289) (end 15.748 23.622) (width 0.635) (layer "F.Cu") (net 5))
 (segment (start 15.748 23.622) (end 16.256 23.114) (width 0.635) (layer "F.Cu") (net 5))
 (segment (start 16.256 23.114) (end 17.0815 23.114) (width 0.635) (layer "F.Cu") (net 5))
 (segment (start 17.0815 23.114) (end 17.2085 23.1075) (width 0.635) (layer "F.Cu") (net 5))
 (segment (start 17.496 26.604) (end 16.063 26.604) (width 0.635) (layer "F.Cu") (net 5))
 (segment (start 17.399 29.464) (end 17.526 29.591) (width 0.3048) (layer "F.Cu") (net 6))
 (segment (start 16.002 29.337) (end 16.4465 29.337) (width 0.254) (layer "F.Cu") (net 6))
 (segment (start 16.0655 29.464) (end 17.399 29.464) (width 0.3048) (layer "F.Cu") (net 6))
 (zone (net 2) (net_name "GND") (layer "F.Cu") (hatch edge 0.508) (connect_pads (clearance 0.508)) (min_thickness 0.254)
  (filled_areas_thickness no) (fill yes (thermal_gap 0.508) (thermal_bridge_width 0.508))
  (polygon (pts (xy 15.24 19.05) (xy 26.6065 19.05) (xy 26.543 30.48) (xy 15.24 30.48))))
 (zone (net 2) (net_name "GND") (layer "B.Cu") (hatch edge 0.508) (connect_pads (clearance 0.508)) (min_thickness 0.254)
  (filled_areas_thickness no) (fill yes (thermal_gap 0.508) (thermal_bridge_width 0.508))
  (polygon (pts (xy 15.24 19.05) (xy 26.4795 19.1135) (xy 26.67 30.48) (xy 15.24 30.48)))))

